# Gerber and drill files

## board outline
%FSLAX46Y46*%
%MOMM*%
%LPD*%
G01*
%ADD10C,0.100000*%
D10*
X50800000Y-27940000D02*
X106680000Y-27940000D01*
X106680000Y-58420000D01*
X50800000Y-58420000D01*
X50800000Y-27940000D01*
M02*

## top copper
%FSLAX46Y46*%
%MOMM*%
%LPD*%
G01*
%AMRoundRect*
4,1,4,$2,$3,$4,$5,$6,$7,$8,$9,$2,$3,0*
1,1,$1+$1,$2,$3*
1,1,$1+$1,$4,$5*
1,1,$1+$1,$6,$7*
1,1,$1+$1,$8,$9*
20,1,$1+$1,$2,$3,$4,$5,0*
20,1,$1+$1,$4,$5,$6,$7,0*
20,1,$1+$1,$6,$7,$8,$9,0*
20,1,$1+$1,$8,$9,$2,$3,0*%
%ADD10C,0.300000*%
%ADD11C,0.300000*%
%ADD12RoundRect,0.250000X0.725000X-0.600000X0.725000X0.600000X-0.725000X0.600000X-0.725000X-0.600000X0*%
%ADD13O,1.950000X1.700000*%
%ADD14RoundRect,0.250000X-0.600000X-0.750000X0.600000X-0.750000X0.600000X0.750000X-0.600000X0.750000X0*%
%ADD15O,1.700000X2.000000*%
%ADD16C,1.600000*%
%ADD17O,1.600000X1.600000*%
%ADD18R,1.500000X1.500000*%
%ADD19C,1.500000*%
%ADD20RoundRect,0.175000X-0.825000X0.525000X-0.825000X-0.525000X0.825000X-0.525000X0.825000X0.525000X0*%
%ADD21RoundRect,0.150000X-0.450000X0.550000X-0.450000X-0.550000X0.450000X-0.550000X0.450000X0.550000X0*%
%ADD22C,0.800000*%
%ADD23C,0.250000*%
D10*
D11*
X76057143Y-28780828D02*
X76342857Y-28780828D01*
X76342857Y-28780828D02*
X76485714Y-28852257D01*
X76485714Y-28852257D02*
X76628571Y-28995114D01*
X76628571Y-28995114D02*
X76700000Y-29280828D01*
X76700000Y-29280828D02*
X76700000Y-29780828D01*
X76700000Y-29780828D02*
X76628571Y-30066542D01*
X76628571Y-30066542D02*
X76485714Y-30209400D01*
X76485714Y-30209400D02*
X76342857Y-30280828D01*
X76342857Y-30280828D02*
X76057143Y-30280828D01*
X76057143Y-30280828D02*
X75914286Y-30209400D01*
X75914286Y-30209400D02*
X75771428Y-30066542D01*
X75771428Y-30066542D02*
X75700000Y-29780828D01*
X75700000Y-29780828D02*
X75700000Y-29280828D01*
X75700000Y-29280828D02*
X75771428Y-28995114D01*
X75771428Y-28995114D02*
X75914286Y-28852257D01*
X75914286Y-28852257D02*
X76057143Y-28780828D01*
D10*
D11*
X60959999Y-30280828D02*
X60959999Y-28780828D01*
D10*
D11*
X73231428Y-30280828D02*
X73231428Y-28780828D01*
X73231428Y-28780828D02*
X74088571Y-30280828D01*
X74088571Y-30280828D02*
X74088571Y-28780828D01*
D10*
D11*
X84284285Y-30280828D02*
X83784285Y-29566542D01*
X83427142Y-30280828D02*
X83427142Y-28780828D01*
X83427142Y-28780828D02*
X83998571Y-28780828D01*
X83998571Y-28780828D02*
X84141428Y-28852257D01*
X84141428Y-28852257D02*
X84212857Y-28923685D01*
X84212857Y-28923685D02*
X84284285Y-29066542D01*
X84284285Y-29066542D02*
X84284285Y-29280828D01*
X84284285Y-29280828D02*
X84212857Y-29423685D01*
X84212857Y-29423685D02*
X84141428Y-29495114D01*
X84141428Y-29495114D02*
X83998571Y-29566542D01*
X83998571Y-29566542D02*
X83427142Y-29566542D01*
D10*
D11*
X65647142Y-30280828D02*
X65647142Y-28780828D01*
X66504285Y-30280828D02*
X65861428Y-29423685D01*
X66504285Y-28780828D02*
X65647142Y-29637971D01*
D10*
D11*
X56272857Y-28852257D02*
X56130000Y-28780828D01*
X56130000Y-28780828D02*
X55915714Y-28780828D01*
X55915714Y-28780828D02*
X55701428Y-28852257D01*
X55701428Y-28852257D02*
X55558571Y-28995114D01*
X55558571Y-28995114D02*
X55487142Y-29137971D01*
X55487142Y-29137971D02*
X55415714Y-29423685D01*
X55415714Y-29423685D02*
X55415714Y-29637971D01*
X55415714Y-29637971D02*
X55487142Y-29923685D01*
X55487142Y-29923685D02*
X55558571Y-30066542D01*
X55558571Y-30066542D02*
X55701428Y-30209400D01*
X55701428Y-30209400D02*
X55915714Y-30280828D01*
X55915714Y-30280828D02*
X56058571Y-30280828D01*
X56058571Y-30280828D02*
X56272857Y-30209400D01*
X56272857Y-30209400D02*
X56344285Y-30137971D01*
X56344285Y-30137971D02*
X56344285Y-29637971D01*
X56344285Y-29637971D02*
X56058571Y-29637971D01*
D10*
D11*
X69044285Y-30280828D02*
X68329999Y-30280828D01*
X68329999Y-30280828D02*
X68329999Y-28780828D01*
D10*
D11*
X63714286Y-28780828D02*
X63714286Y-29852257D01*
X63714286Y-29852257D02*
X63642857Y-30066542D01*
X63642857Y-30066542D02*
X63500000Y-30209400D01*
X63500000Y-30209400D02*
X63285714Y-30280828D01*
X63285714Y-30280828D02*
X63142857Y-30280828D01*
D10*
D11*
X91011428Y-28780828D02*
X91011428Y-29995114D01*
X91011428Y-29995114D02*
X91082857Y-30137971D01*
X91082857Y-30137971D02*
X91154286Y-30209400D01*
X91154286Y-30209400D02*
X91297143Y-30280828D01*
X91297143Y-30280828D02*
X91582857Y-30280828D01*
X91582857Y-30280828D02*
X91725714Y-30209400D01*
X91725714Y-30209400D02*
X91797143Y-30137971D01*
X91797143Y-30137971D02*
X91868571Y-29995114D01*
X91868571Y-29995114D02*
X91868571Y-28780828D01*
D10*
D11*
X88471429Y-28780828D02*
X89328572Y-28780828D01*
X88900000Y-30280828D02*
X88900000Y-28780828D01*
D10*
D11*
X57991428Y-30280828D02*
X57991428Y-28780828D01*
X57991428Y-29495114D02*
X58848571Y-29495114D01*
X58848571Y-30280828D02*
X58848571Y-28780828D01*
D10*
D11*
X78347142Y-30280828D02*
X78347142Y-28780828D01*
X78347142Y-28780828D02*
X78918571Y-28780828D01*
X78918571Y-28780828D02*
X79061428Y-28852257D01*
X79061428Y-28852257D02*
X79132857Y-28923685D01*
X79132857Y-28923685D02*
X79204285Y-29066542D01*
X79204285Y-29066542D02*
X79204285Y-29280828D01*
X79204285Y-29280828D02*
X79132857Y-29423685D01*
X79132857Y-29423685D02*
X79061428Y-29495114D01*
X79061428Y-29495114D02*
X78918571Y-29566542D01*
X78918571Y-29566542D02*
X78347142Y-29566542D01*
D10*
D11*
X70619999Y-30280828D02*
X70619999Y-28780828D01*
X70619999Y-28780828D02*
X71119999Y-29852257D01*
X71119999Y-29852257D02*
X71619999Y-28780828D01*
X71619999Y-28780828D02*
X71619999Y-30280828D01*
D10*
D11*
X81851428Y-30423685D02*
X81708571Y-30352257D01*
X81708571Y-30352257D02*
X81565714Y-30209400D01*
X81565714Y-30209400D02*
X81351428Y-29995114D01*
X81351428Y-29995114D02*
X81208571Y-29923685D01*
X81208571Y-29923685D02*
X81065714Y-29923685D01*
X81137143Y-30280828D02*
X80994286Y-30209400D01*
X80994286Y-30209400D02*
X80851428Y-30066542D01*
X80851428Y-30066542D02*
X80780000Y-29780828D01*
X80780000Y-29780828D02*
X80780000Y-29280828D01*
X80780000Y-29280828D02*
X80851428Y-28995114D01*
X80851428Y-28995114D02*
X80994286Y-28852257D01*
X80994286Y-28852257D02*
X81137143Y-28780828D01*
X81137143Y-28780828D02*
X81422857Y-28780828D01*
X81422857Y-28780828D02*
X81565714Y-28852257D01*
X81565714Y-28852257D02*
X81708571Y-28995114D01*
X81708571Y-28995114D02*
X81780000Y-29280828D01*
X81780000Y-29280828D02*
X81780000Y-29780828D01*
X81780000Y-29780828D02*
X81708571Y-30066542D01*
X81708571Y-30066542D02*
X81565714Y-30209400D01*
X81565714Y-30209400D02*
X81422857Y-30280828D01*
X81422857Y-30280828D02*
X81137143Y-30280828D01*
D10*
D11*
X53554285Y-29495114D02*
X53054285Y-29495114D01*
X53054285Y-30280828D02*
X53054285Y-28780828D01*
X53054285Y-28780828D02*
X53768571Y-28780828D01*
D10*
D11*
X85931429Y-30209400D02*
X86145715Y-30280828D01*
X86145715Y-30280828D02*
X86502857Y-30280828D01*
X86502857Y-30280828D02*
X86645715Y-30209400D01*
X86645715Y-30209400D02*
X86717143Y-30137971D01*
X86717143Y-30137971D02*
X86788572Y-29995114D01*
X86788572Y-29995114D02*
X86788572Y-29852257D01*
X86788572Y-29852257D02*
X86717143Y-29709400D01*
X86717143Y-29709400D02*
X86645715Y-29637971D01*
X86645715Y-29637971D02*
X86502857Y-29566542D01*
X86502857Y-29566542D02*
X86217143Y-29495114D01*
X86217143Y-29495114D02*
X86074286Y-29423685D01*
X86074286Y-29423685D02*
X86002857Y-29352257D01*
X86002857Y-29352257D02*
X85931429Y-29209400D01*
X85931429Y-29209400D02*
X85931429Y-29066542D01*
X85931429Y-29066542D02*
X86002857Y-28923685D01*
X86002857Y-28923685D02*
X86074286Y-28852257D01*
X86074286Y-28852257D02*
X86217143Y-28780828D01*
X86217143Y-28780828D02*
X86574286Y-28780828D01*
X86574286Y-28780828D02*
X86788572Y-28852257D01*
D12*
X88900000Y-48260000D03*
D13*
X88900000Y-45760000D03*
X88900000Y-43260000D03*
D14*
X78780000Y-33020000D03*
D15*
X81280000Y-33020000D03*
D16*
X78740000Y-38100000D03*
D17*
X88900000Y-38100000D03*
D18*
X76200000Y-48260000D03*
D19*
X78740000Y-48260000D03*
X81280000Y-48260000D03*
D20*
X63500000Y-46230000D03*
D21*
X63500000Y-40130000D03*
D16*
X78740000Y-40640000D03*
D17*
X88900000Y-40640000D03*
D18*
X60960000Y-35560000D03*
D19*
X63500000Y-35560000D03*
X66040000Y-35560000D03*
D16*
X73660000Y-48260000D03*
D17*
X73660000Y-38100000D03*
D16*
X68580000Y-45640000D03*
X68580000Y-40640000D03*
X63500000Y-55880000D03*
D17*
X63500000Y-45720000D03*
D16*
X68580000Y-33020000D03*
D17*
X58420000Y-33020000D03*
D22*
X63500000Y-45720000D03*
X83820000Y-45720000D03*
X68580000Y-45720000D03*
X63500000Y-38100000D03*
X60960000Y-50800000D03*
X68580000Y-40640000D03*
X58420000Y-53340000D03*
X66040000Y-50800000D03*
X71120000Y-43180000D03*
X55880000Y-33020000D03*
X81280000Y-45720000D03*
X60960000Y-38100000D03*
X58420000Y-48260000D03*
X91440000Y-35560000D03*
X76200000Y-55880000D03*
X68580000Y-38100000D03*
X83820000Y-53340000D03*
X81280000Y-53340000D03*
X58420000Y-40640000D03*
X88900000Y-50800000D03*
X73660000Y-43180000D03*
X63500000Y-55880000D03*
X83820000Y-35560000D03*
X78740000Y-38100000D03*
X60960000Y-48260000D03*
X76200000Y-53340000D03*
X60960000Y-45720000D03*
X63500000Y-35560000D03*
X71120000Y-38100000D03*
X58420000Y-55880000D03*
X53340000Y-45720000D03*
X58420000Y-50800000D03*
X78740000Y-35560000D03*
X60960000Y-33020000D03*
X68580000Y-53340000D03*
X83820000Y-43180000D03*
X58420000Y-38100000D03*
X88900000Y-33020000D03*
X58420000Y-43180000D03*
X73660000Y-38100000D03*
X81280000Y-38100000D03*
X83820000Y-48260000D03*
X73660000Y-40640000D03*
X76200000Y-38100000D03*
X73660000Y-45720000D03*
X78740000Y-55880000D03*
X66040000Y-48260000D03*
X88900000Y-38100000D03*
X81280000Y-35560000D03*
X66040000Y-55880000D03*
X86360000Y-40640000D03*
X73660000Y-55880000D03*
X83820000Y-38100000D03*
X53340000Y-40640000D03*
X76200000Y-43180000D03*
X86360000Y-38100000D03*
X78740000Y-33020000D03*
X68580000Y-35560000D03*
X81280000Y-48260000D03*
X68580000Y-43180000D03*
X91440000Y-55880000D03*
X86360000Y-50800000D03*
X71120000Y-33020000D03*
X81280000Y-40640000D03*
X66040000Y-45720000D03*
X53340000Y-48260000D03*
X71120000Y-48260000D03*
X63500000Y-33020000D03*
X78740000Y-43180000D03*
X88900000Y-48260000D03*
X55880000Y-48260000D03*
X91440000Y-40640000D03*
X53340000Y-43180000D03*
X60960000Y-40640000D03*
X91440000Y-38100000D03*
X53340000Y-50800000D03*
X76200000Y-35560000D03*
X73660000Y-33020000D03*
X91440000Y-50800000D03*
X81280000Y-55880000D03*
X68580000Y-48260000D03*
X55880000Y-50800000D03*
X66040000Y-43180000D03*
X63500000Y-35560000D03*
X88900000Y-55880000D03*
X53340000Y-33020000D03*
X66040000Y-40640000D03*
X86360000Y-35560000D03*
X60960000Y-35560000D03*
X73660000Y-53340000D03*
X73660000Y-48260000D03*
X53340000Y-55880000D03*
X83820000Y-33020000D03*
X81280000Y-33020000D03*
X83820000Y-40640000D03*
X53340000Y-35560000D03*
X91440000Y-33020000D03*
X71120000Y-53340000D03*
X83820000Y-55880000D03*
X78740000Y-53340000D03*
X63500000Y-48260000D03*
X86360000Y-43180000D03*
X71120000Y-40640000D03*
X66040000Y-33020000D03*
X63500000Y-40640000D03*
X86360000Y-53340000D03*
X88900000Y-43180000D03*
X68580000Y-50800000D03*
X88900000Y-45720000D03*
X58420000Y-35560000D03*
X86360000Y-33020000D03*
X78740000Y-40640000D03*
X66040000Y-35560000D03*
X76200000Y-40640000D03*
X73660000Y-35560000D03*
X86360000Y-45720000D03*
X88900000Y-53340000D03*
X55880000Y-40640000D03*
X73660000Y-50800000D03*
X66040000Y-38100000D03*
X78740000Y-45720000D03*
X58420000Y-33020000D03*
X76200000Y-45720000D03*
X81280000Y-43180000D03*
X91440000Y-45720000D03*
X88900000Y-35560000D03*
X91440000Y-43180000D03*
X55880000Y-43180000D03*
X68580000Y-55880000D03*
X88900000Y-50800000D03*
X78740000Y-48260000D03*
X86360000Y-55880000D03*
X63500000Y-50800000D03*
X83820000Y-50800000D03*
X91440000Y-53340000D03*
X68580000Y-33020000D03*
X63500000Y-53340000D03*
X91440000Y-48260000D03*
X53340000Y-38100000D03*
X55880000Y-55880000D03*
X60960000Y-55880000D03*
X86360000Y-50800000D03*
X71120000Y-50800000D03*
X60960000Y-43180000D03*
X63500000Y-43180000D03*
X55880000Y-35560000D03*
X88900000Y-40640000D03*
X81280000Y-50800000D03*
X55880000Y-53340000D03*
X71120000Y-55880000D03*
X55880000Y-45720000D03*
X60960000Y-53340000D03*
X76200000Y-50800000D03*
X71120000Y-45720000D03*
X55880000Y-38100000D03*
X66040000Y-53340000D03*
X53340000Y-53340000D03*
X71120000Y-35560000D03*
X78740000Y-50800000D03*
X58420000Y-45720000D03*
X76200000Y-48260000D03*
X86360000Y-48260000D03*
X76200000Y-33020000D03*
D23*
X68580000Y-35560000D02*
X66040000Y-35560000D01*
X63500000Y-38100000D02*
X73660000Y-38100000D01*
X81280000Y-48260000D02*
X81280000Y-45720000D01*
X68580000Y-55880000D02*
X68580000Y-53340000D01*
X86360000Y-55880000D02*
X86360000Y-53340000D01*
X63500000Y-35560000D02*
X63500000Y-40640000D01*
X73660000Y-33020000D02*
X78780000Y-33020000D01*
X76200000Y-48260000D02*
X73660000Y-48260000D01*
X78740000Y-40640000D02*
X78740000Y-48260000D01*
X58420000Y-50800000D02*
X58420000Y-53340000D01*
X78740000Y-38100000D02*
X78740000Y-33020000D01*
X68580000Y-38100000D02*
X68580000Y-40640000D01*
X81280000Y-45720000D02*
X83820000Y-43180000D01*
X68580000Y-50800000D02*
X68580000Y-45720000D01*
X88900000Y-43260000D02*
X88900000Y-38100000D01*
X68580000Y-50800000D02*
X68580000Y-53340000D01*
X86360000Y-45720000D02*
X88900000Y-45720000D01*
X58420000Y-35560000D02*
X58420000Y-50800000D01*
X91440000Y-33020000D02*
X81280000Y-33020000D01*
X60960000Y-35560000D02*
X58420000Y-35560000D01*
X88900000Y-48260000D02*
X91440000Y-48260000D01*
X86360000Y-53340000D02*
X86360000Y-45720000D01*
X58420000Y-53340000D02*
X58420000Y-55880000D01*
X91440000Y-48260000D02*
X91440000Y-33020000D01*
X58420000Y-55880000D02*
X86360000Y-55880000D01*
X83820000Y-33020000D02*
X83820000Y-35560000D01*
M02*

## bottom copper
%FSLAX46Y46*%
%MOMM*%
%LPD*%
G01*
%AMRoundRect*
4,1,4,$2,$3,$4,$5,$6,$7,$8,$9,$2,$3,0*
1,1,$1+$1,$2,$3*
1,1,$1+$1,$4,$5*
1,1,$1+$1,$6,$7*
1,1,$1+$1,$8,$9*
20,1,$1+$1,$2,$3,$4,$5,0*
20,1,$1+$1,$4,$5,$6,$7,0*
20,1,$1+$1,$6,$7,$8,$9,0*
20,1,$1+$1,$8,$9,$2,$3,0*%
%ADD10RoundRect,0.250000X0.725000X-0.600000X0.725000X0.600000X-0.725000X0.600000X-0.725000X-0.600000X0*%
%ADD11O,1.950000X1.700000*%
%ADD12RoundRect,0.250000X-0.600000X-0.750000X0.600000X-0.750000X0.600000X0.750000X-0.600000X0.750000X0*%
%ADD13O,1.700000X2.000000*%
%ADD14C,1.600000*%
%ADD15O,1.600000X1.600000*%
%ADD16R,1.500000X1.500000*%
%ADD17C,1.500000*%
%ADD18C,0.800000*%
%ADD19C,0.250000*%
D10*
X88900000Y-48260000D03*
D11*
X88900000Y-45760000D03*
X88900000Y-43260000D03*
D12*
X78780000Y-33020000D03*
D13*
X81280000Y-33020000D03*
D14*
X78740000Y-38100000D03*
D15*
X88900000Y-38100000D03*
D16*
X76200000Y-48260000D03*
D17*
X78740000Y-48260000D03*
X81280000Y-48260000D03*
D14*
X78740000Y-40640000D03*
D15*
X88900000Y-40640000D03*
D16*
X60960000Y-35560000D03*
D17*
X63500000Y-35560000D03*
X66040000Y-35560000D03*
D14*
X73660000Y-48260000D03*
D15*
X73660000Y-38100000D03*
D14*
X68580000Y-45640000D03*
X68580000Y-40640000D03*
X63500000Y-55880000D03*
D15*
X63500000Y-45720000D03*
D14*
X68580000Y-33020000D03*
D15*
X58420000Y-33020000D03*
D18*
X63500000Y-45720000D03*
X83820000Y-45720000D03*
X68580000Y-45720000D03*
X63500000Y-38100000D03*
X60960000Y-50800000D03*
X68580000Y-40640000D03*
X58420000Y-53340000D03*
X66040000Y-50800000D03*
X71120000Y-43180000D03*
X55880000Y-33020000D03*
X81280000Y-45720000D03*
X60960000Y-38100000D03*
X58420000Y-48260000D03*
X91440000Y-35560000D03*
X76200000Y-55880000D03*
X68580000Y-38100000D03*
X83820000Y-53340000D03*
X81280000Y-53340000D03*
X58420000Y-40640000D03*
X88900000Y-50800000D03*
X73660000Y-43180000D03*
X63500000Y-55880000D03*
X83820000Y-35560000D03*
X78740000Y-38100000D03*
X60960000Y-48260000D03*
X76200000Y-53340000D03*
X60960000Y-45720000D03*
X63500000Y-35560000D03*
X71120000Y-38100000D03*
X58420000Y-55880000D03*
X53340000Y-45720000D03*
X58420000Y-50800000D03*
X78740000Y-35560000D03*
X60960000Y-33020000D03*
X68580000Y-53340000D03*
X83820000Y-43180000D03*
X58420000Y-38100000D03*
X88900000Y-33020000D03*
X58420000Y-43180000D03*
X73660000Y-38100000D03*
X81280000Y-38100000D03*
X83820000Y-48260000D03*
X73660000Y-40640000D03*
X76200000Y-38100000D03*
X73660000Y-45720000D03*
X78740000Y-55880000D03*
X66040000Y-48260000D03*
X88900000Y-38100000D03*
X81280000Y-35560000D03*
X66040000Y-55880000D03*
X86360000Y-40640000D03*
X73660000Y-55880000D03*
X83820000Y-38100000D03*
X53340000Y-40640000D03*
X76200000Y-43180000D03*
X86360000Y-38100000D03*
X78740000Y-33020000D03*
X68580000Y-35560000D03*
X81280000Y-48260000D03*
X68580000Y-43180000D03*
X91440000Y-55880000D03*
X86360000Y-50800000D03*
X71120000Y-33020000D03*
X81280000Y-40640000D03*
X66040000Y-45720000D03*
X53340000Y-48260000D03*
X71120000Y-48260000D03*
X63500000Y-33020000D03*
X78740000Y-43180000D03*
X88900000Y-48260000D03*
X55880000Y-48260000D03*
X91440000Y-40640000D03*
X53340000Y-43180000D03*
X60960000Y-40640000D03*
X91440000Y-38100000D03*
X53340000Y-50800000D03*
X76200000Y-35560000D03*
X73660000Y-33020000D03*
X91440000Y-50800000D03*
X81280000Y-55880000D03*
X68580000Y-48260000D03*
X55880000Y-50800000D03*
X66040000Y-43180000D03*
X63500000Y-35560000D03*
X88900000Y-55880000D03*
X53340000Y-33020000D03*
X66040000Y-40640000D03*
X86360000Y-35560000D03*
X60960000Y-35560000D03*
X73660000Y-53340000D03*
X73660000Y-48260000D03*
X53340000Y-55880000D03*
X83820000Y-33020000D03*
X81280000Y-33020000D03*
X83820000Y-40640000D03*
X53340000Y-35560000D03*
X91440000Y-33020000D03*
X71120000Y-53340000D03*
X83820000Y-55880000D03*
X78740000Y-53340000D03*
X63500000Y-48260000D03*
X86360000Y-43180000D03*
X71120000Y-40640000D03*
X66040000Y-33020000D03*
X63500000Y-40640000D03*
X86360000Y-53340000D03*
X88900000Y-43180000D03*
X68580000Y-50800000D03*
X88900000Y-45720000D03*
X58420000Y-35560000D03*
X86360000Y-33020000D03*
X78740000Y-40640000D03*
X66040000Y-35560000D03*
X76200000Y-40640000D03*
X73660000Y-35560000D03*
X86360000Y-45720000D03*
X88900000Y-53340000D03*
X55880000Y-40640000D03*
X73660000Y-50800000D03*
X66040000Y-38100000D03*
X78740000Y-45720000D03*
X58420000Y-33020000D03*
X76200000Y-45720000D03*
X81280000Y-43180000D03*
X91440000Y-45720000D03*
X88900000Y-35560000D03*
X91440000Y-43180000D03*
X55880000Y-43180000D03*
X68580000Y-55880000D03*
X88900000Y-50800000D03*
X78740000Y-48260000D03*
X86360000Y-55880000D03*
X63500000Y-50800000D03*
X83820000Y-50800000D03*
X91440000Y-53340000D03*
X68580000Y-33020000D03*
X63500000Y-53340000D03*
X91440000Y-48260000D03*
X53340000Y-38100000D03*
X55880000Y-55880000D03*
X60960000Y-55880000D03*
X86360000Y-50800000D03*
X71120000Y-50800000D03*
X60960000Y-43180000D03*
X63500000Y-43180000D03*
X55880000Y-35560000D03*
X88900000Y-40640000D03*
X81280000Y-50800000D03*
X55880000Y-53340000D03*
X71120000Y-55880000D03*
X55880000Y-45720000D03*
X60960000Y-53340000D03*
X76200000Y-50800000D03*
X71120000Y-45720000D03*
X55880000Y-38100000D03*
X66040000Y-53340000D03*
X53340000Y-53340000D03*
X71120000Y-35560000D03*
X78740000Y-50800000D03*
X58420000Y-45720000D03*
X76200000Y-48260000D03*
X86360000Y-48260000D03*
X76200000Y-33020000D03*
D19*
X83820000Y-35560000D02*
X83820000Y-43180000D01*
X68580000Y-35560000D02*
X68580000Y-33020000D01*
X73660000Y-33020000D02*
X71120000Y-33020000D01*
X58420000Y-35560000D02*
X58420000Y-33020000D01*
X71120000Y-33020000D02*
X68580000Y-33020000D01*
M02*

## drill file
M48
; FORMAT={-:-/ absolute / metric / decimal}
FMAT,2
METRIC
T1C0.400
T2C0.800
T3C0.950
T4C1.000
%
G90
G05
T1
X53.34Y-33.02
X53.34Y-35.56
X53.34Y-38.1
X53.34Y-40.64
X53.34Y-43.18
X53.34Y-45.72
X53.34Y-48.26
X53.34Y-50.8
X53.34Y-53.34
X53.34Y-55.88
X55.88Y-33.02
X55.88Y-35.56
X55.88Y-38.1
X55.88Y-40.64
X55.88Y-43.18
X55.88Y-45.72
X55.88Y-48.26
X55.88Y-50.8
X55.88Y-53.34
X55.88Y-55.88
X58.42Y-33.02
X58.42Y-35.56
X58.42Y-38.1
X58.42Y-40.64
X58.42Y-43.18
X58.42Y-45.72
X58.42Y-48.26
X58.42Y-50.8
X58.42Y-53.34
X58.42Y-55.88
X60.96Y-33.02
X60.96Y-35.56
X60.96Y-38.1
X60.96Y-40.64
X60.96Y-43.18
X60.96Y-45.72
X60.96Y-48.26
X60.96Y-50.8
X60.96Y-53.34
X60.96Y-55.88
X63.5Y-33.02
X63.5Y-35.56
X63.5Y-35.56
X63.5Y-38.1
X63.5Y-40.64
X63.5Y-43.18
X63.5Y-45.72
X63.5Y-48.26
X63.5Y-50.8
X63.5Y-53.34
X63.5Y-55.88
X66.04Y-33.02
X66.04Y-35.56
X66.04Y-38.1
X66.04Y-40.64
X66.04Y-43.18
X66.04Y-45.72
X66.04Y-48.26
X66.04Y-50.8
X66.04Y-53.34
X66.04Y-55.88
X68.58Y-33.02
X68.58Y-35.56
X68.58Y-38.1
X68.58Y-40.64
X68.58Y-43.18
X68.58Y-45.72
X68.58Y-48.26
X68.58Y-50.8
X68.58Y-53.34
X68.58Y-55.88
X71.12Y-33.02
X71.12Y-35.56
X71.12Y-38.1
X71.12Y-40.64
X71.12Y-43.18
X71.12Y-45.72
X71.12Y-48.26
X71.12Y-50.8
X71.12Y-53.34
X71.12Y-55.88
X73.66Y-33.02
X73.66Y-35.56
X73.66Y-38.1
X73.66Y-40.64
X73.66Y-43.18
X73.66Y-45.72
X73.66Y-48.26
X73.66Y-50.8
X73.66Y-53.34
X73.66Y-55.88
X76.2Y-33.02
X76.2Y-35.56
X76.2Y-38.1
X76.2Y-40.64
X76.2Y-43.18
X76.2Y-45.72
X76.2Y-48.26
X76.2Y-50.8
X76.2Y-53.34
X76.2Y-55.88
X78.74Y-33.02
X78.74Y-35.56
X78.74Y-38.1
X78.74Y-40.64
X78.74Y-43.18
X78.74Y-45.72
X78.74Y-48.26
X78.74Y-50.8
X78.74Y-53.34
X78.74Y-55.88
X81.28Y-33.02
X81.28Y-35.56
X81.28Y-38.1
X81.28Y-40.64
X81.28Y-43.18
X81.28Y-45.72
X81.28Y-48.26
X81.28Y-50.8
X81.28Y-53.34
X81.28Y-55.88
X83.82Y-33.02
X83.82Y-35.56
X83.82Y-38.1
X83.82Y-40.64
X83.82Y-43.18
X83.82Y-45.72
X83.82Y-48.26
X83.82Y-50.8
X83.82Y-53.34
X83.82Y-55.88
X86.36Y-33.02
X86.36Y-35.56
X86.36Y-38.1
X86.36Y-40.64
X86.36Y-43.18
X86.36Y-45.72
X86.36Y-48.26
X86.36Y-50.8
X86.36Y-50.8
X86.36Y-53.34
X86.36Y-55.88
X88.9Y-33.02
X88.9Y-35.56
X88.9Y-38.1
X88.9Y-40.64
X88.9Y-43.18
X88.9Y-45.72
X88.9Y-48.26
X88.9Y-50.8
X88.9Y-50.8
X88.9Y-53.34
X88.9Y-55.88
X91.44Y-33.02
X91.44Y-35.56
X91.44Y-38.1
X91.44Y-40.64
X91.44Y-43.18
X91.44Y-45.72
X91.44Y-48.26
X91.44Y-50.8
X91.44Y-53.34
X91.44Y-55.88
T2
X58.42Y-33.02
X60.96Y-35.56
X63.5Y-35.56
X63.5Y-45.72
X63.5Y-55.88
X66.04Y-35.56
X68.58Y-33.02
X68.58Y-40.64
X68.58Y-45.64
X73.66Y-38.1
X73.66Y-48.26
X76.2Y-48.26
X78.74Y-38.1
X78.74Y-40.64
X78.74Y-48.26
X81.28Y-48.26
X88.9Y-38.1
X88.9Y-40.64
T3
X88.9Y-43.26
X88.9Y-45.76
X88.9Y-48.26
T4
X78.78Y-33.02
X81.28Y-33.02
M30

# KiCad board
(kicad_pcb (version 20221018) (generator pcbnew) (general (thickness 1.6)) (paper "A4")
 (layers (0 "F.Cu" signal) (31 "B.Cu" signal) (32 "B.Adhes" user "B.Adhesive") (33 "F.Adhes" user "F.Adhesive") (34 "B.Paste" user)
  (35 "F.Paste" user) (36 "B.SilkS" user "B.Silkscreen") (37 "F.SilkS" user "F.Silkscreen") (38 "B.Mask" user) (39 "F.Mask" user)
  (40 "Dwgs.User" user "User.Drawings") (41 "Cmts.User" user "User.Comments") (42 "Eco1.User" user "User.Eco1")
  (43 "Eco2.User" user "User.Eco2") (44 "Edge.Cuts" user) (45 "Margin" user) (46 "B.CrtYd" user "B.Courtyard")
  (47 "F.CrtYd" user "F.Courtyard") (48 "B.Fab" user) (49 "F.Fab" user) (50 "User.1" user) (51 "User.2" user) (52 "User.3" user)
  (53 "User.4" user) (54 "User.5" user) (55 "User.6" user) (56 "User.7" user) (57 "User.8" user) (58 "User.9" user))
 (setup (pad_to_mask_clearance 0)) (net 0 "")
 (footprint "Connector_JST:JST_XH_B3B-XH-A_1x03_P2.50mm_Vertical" (layer "F.Cu") (at 88.9 48.26 90)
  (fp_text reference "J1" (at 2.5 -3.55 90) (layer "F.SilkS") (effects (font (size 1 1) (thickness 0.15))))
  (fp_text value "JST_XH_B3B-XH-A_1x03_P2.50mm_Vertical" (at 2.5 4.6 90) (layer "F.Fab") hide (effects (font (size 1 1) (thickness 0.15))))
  (pad "1" thru_hole roundrect (at 0 0 90) (size 1.7 1.95) (drill 0.95) (layers "*.Cu" "*.Mask") (roundrect_rratio 0.147059))
  (pad "2" thru_hole oval (at 2.5 0 90) (size 1.7 1.95) (drill 0.95) (layers "*.Cu" "*.Mask"))
  (pad "3" thru_hole oval (at 5 0 90) (size 1.7 1.95) (drill 0.95) (layers "*.Cu" "*.Mask")))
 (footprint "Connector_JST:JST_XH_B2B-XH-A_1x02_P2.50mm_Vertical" (layer "F.Cu") (at 78.78 33.02)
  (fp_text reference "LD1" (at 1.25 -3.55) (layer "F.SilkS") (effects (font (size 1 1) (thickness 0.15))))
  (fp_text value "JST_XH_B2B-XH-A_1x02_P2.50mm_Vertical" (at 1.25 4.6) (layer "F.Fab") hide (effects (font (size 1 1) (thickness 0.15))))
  (pad "1" thru_hole roundrect (at 0 0) (size 1.7 2) (drill 1) (layers "*.Cu" "*.Mask") (roundrect_rratio 0.147059))
  (pad "2" thru_hole oval (at 2.5 0) (size 1.7 2) (drill 1) (layers "*.Cu" "*.Mask")))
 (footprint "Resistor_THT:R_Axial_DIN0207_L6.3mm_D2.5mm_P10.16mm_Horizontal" (layer "F.Cu") (at 78.74 38.1)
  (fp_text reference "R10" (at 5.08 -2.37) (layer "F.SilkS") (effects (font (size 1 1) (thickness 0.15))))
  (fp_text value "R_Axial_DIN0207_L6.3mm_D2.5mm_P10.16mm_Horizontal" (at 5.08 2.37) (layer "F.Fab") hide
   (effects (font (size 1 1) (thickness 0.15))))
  (pad "1" thru_hole circle (at 0 0) (size 1.6 1.6) (drill 0.8) (layers "*.Cu" "*.Mask"))
  (pad "2" thru_hole oval (at 10.16 0) (size 1.6 1.6) (drill 0.8) (layers "*.Cu" "*.Mask")))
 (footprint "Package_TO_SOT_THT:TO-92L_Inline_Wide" (layer "F.Cu") (at 76.2 48.26)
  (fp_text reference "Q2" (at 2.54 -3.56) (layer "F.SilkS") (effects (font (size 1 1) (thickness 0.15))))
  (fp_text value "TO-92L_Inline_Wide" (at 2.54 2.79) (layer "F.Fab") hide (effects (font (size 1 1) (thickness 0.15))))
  (pad "1" thru_hole rect (at 0 0) (size 1.5 1.5) (drill 0.8) (layers "*.Cu" "*.Mask"))
  (pad "2" thru_hole circle (at 2.54 0) (size 1.5 1.5) (drill 0.8) (layers "*.Cu" "*.Mask"))
  (pad "3" thru_hole circle (at 5.08 0) (size 1.5 1.5) (drill 0.8) (layers "*.Cu" "*.Mask")))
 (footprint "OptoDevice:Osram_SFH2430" (layer "F.Cu") (at 63.5 43.18 90)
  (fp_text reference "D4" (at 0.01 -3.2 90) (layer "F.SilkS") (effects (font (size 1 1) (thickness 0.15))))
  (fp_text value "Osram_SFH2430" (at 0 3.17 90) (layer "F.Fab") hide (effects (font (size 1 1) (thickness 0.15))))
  (pad "" smd roundrect (at -3.05 0 270) (size 1.3 1.9) (layers "F.Paste") (roundrect_rratio 0.125))
  (pad "" smd roundrect (at -3.05 0 270) (size 1.5 2.1) (layers "F.Mask") (roundrect_rratio 0.125))
  (pad "" smd roundrect (at 3.05 0 270) (size 1.3 1.1) (layers "F.Paste") (roundrect_rratio 0.125))
  (pad "" smd roundrect (at 3.05 0 270) (size 1.5 1.3) (layers "F.Mask") (roundrect_rratio 0.125))
  (pad "1" smd roundrect (at -3.05 0 270) (size 1.4 2) (layers "F.Cu" "F.Mask") (roundrect_rratio 0.125))
  (pad "2" smd roundrect (at 3.05 0 270) (size 1.4 1.2) (layers "F.Cu" "F.Mask") (roundrect_rratio 0.125)))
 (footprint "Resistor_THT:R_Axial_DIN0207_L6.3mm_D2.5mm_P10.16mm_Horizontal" (layer "F.Cu") (at 78.74 40.64)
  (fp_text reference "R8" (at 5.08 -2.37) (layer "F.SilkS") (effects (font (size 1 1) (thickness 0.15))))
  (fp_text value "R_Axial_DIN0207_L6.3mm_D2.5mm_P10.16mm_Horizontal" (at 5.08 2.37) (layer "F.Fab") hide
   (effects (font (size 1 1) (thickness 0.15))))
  (pad "1" thru_hole circle (at 0 0) (size 1.6 1.6) (drill 0.8) (layers "*.Cu" "*.Mask"))
  (pad "2" thru_hole oval (at 10.16 0) (size 1.6 1.6) (drill 0.8) (layers "*.Cu" "*.Mask")))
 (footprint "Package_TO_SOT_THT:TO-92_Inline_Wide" (layer "F.Cu") (at 60.96 35.56)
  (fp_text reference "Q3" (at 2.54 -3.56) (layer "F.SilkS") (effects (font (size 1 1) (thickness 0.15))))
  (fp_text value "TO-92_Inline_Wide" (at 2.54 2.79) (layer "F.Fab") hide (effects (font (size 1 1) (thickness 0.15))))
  (pad "1" thru_hole rect (at 0 0) (size 1.5 1.5) (drill 0.8) (layers "*.Cu" "*.Mask"))
  (pad "2" thru_hole circle (at 2.54 0) (size 1.5 1.5) (drill 0.8) (layers "*.Cu" "*.Mask"))
  (pad "3" thru_hole circle (at 5.08 0) (size 1.5 1.5) (drill 0.8) (layers "*.Cu" "*.Mask")))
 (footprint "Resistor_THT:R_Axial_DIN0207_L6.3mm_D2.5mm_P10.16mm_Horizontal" (layer "B.Cu") (at 73.66 48.26 90)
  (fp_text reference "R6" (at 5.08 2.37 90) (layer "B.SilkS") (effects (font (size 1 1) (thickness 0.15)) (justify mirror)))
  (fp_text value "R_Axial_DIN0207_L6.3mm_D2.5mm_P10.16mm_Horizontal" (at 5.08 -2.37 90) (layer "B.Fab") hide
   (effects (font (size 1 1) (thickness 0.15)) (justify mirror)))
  (pad "1" thru_hole circle (at 0 0 90) (size 1.6 1.6) (drill 0.8) (layers "*.Cu" "*.Mask"))
  (pad "2" thru_hole oval (at 10.16 0 90) (size 1.6 1.6) (drill 0.8) (layers "*.Cu" "*.Mask")))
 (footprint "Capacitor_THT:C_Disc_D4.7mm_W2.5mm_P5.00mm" (layer "B.Cu") (at 68.58 45.64 90)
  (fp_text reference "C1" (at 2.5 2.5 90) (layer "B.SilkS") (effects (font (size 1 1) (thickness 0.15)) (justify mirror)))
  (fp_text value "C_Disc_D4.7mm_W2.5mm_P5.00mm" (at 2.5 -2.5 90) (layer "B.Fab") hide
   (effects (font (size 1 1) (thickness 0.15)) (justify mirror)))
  (pad "1" thru_hole circle (at 0 0 90) (size 1.6 1.6) (drill 0.8) (layers "*.Cu" "*.Mask"))
  (pad "2" thru_hole circle (at 5 0 90) (size 1.6 1.6) (drill 0.8) (layers "*.Cu" "*.Mask")))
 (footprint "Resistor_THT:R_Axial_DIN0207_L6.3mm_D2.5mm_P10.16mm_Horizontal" (layer "B.Cu") (at 63.5 55.88 90)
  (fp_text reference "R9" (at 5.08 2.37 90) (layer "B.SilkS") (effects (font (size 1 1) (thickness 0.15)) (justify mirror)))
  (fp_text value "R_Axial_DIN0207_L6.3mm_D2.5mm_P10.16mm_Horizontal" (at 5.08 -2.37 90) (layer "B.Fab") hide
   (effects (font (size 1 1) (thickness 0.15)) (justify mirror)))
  (pad "1" thru_hole circle (at 0 0 90) (size 1.6 1.6) (drill 0.8) (layers "*.Cu" "*.Mask"))
  (pad "2" thru_hole oval (at 10.16 0 90) (size 1.6 1.6) (drill 0.8) (layers "*.Cu" "*.Mask")))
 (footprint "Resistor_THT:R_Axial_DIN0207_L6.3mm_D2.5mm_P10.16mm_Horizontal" (layer "B.Cu") (at 68.58 33.02 180)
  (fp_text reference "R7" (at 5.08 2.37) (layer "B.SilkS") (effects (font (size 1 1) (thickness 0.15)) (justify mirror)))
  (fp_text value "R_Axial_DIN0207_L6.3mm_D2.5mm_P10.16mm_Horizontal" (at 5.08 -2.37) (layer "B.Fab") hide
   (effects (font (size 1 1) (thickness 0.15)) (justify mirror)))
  (pad "1" thru_hole circle (at 0 0 180) (size 1.6 1.6) (drill 0.8) (layers "*.Cu" "*.Mask"))
  (pad "2" thru_hole oval (at 10.16 0 180) (size 1.6 1.6) (drill 0.8) (layers "*.Cu" "*.Mask")))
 (gr_rect (start 50.8 27.94) (end 106.68 58.42) (stroke (width 0.1) (type default)) (fill none) (layer "Edge.Cuts"))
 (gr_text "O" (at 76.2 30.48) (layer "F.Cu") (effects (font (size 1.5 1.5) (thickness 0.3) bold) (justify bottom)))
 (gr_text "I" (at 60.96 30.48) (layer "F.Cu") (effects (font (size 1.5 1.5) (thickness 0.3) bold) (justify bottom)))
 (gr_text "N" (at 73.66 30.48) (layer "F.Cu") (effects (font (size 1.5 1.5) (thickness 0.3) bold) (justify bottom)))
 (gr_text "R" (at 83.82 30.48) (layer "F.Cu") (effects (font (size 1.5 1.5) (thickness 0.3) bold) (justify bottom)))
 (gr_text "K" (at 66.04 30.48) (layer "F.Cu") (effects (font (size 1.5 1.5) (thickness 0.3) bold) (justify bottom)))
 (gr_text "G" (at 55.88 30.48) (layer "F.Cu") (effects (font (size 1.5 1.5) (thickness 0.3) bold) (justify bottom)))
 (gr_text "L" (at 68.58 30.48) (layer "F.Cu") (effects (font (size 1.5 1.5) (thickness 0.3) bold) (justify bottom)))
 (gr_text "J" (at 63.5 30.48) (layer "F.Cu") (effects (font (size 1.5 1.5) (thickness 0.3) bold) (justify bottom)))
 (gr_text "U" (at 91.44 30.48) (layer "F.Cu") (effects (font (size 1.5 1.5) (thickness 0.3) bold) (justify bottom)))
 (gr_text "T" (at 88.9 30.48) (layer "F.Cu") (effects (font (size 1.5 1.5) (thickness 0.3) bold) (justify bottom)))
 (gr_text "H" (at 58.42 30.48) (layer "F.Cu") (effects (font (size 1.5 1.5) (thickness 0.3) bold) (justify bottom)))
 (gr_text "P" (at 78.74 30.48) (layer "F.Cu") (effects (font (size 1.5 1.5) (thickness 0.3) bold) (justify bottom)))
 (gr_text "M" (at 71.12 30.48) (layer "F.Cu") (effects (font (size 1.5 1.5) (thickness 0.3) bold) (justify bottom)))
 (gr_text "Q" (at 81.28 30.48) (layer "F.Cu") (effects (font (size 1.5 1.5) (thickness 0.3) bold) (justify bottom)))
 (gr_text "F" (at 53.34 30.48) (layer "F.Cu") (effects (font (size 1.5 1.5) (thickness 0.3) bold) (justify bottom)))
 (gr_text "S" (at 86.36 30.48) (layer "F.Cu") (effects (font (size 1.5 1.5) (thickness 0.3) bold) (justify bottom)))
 (segment (start 68.58 35.56) (end 66.04 35.56) (width 0.25) (layer "F.Cu") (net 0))
 (segment (start 63.5 38.1) (end 73.66 38.1) (width 0.25) (layer "F.Cu") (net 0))
 (segment (start 81.28 48.26) (end 81.28 45.72) (width 0.25) (layer "F.Cu") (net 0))
 (segment (start 68.58 55.88) (end 68.58 53.34) (width 0.25) (layer "F.Cu") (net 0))
 (segment (start 86.36 55.88) (end 86.36 53.34) (width 0.25) (layer "F.Cu") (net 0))
 (segment (start 63.5 35.56) (end 63.5 40.64) (width 0.25) (layer "F.Cu") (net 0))
 (segment (start 73.66 33.02) (end 78.78 33.02) (width 0.25) (layer "F.Cu") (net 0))
 (segment (start 76.2 48.26) (end 73.66 48.26) (width 0.25) (layer "F.Cu") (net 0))
 (segment (start 78.74 40.64) (end 78.74 48.26) (width 0.25) (layer "F.Cu") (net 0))
 (segment (start 58.42 50.8) (end 58.42 53.34) (width 0.25) (layer "F.Cu") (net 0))
 (segment (start 78.74 38.1) (end 78.74 33.02) (width 0.25) (layer "F.Cu") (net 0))
 (segment (start 68.58 38.1) (end 68.58 40.64) (width 0.25) (layer "F.Cu") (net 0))
 (segment (start 81.28 45.72) (end 83.82 43.18) (width 0.25) (layer "F.Cu") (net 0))
 (segment (start 68.58 50.8) (end 68.58 45.72) (width 0.25) (layer "F.Cu") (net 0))
 (segment (start 88.9 43.26) (end 88.9 38.1) (width 0.25) (layer "F.Cu") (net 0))
 (segment (start 68.58 50.8) (end 68.58 53.34) (width 0.25) (layer "F.Cu") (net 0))
 (segment (start 86.36 45.72) (end 88.9 45.72) (width 0.25) (layer "F.Cu") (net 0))
 (segment (start 58.42 35.56) (end 58.42 50.8) (width 0.25) (layer "F.Cu") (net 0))
 (segment (start 91.44 33.02) (end 81.28 33.02) (width 0.25) (layer "F.Cu") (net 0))
 (segment (start 60.96 35.56) (end 58.42 35.56) (width 0.25) (layer "F.Cu") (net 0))
 (segment (start 88.9 48.26) (end 91.44 48.26) (width 0.25) (layer "F.Cu") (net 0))
 (segment (start 86.36 53.34) (end 86.36 45.72) (width 0.25) (layer "F.Cu") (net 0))
 (segment (start 58.42 53.34) (end 58.42 55.88) (width 0.25) (layer "F.Cu") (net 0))
 (segment (start 91.44 48.26) (end 91.44 33.02) (width 0.25) (layer "F.Cu") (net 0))
 (segment (start 58.42 55.88) (end 86.36 55.88) (width 0.25) (layer "F.Cu") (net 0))
 (segment (start 83.82 33.02) (end 83.82 35.56) (width 0.25) (layer "F.Cu") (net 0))
 (via (at 63.5 45.72) (size 0.8) (drill 0.4) (layers "F.Cu" "B.Cu") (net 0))
 (via (at 83.82 45.72) (size 0.8) (drill 0.4) (layers "F.Cu" "B.Cu") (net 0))
 (via (at 68.58 45.72) (size 0.8) (drill 0.4) (layers "F.Cu" "B.Cu") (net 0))
 (via (at 63.5 38.1) (size 0.8) (drill 0.4) (layers "F.Cu" "B.Cu") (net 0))
 (via (at 60.96 50.8) (size 0.8) (drill 0.4) (layers "F.Cu" "B.Cu") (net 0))
 (via (at 68.58 40.64) (size 0.8) (drill 0.4) (layers "F.Cu" "B.Cu") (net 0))
 (via (at 58.42 53.34) (size 0.8) (drill 0.4) (layers "F.Cu" "B.Cu") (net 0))
 (via (at 66.04 50.8) (size 0.8) (drill 0.4) (layers "F.Cu" "B.Cu") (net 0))
 (via (at 71.12 43.18) (size 0.8) (drill 0.4) (layers "F.Cu" "B.Cu") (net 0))
 (via (at 55.88 33.02) (size 0.8) (drill 0.4) (layers "F.Cu" "B.Cu") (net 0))
 (via (at 81.28 45.72) (size 0.8) (drill 0.4) (layers "F.Cu" "B.Cu") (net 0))
 (via (at 60.96 38.1) (size 0.8) (drill 0.4) (layers "F.Cu" "B.Cu") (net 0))
 (via (at 58.42 48.26) (size 0.8) (drill 0.4) (layers "F.Cu" "B.Cu") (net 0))
 (via (at 91.44 35.56) (size 0.8) (drill 0.4) (layers "F.Cu" "B.Cu") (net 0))
 (via (at 76.2 55.88) (size 0.8) (drill 0.4) (layers "F.Cu" "B.Cu") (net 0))
 (via (at 68.58 38.1) (size 0.8) (drill 0.4) (layers "F.Cu" "B.Cu") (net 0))
 (via (at 83.82 53.34) (size 0.8) (drill 0.4) (layers "F.Cu" "B.Cu") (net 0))
 (via (at 81.28 53.34) (size 0.8) (drill 0.4) (layers "F.Cu" "B.Cu") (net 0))
 (via (at 58.42 40.64) (size 0.8) (drill 0.4) (layers "F.Cu" "B.Cu") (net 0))
 (via (at 88.9 50.8) (size 0.8) (drill 0.4) (layers "F.Cu" "B.Cu") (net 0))
 (via (at 73.66 43.18) (size 0.8) (drill 0.4) (layers "F.Cu" "B.Cu") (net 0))
 (via (at 63.5 55.88) (size 0.8) (drill 0.4) (layers "F.Cu" "B.Cu") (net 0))
 (via (at 83.82 35.56) (size 0.8) (drill 0.4) (layers "F.Cu" "B.Cu") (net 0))
 (via (at 78.74 38.1) (size 0.8) (drill 0.4) (layers "F.Cu" "B.Cu") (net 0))
 (via (at 60.96 48.26) (size 0.8) (drill 0.4) (layers "F.Cu" "B.Cu") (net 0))
 (via (at 76.2 53.34) (size 0.8) (drill 0.4) (layers "F.Cu" "B.Cu") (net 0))
 (via (at 60.96 45.72) (size 0.8) (drill 0.4) (layers "F.Cu" "B.Cu") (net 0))
 (via (at 63.5 35.56) (size 0.8) (drill 0.4) (layers "F.Cu" "B.Cu") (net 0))
 (via (at 71.12 38.1) (size 0.8) (drill 0.4) (layers "F.Cu" "B.Cu") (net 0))
 (via (at 58.42 55.88) (size 0.8) (drill 0.4) (layers "F.Cu" "B.Cu") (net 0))
 (via (at 53.34 45.72) (size 0.8) (drill 0.4) (layers "F.Cu" "B.Cu") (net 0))
 (via (at 58.42 50.8) (size 0.8) (drill 0.4) (layers "F.Cu" "B.Cu") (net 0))
 (via (at 78.74 35.56) (size 0.8) (drill 0.4) (layers "F.Cu" "B.Cu") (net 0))
 (via (at 60.96 33.02) (size 0.8) (drill 0.4) (layers "F.Cu" "B.Cu") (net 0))
 (via (at 68.58 53.34) (size 0.8) (drill 0.4) (layers "F.Cu" "B.Cu") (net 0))
 (via (at 83.82 43.18) (size 0.8) (drill 0.4) (layers "F.Cu" "B.Cu") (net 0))
 (via (at 58.42 38.1) (size 0.8) (drill 0.4) (layers "F.Cu" "B.Cu") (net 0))
 (via (at 88.9 33.02) (size 0.8) (drill 0.4) (layers "F.Cu" "B.Cu") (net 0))
 (via (at 58.42 43.18) (size 0.8) (drill 0.4) (layers "F.Cu" "B.Cu") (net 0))
 (via (at 73.66 38.1) (size 0.8) (drill 0.4) (layers "F.Cu" "B.Cu") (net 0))
 (via (at 81.28 38.1) (size 0.8) (drill 0.4) (layers "F.Cu" "B.Cu") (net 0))
 (via (at 83.82 48.26) (size 0.8) (drill 0.4) (layers "F.Cu" "B.Cu") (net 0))
 (via (at 73.66 40.64) (size 0.8) (drill 0.4) (layers "F.Cu" "B.Cu") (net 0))
 (via (at 76.2 38.1) (size 0.8) (drill 0.4) (layers "F.Cu" "B.Cu") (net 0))
 (via (at 73.66 45.72) (size 0.8) (drill 0.4) (layers "F.Cu" "B.Cu") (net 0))
 (via (at 78.74 55.88) (size 0.8) (drill 0.4) (layers "F.Cu" "B.Cu") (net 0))
 (via (at 66.04 48.26) (size 0.8) (drill 0.4) (layers "F.Cu" "B.Cu") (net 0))
 (via (at 88.9 38.1) (size 0.8) (drill 0.4) (layers "F.Cu" "B.Cu") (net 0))
 (via (at 81.28 35.56) (size 0.8) (drill 0.4) (layers "F.Cu" "B.Cu") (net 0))
 (via (at 66.04 55.88) (size 0.8) (drill 0.4) (layers "F.Cu" "B.Cu") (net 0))
 (via (at 86.36 40.64) (size 0.8) (drill 0.4) (layers "F.Cu" "B.Cu") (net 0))
 (via (at 73.66 55.88) (size 0.8) (drill 0.4) (layers "F.Cu" "B.Cu") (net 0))
 (via (at 83.82 38.1) (size 0.8) (drill 0.4) (layers "F.Cu" "B.Cu") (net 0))
 (via (at 53.34 40.64) (size 0.8) (drill 0.4) (layers "F.Cu" "B.Cu") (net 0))
 (via (at 76.2 43.18) (size 0.8) (drill 0.4) (layers "F.Cu" "B.Cu") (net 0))
 (via (at 86.36 38.1) (size 0.8) (drill 0.4) (layers "F.Cu" "B.Cu") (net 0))
 (via (at 78.74 33.02) (size 0.8) (drill 0.4) (layers "F.Cu" "B.Cu") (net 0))
 (via (at 68.58 35.56) (size 0.8) (drill 0.4) (layers "F.Cu" "B.Cu") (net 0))
 (via (at 81.28 48.26) (size 0.8) (drill 0.4) (layers "F.Cu" "B.Cu") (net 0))
 (via (at 68.58 43.18) (size 0.8) (drill 0.4) (layers "F.Cu" "B.Cu") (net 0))
 (via (at 91.44 55.88) (size 0.8) (drill 0.4) (layers "F.Cu" "B.Cu") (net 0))
 (via (at 86.36 50.8) (size 0.8) (drill 0.4) (layers "F.Cu" "B.Cu") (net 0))
 (via (at 71.12 33.02) (size 0.8) (drill 0.4) (layers "F.Cu" "B.Cu") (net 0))
 (via (at 81.28 40.64) (size 0.8) (drill 0.4) (layers "F.Cu" "B.Cu") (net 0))
 (via (at 66.04 45.72) (size 0.8) (drill 0.4) (layers "F.Cu" "B.Cu") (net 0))
 (via (at 53.34 48.26) (size 0.8) (drill 0.4) (layers "F.Cu" "B.Cu") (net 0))
 (via (at 71.12 48.26) (size 0.8) (drill 0.4) (layers "F.Cu" "B.Cu") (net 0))
 (via (at 63.5 33.02) (size 0.8) (drill 0.4) (layers "F.Cu" "B.Cu") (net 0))
 (via (at 78.74 43.18) (size 0.8) (drill 0.4) (layers "F.Cu" "B.Cu") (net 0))
 (via (at 88.9 48.26) (size 0.8) (drill 0.4) (layers "F.Cu" "B.Cu") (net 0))
 (via (at 55.88 48.26) (size 0.8) (drill 0.4) (layers "F.Cu" "B.Cu") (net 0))
 (via (at 91.44 40.64) (size 0.8) (drill 0.4) (layers "F.Cu" "B.Cu") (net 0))
 (via (at 53.34 43.18) (size 0.8) (drill 0.4) (layers "F.Cu" "B.Cu") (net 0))
 (via (at 60.96 40.64) (size 0.8) (drill 0.4) (layers "F.Cu" "B.Cu") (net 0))
 (via (at 91.44 38.1) (size 0.8) (drill 0.4) (layers "F.Cu" "B.Cu") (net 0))
 (via (at 53.34 50.8) (size 0.8) (drill 0.4) (layers "F.Cu" "B.Cu") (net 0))
 (via (at 76.2 35.56) (size 0.8) (drill 0.4) (layers "F.Cu" "B.Cu") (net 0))
 (via (at 73.66 33.02) (size 0.8) (drill 0.4) (layers "F.Cu" "B.Cu") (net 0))
 (via (at 91.44 50.8) (size 0.8) (drill 0.4) (layers "F.Cu" "B.Cu") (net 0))
 (via (at 81.28 55.88) (size 0.8) (drill 0.4) (layers "F.Cu" "B.Cu") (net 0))
 (via (at 68.58 48.26) (size 0.8) (drill 0.4) (layers "F.Cu" "B.Cu") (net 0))
 (via (at 55.88 50.8) (size 0.8) (drill 0.4) (layers "F.Cu" "B.Cu") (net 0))
 (via (at 66.04 43.18) (size 0.8) (drill 0.4) (layers "F.Cu" "B.Cu") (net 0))
 (via (at 63.5 35.56) (size 0.8) (drill 0.4) (layers "F.Cu" "B.Cu") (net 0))
 (via (at 88.9 55.88) (size 0.8) (drill 0.4) (layers "F.Cu" "B.Cu") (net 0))
 (via (at 53.34 33.02) (size 0.8) (drill 0.4) (layers "F.Cu" "B.Cu") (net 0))
 (via (at 66.04 40.64) (size 0.8) (drill 0.4) (layers "F.Cu" "B.Cu") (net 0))
 (via (at 86.36 35.56) (size 0.8) (drill 0.4) (layers "F.Cu" "B.Cu") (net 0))
 (via (at 60.96 35.56) (size 0.8) (drill 0.4) (layers "F.Cu" "B.Cu") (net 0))
 (via (at 73.66 53.34) (size 0.8) (drill 0.4) (layers "F.Cu" "B.Cu") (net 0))
 (via (at 73.66 48.26) (size 0.8) (drill 0.4) (layers "F.Cu" "B.Cu") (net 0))
 (via (at 53.34 55.88) (size 0.8) (drill 0.4) (layers "F.Cu" "B.Cu") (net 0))
 (via (at 83.82 33.02) (size 0.8) (drill 0.4) (layers "F.Cu" "B.Cu") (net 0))
 (via (at 81.28 33.02) (size 0.8) (drill 0.4) (layers "F.Cu" "B.Cu") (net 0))
 (via (at 83.82 40.64) (size 0.8) (drill 0.4) (layers "F.Cu" "B.Cu") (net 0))
 (via (at 53.34 35.56) (size 0.8) (drill 0.4) (layers "F.Cu" "B.Cu") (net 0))
 (via (at 91.44 33.02) (size 0.8) (drill 0.4) (layers "F.Cu" "B.Cu") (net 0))
 (via (at 71.12 53.34) (size 0.8) (drill 0.4) (layers "F.Cu" "B.Cu") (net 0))
 (via (at 83.82 55.88) (size 0.8) (drill 0.4) (layers "F.Cu" "B.Cu") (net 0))
 (via (at 78.74 53.34) (size 0.8) (drill 0.4) (layers "F.Cu" "B.Cu") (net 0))
 (via (at 63.5 48.26) (size 0.8) (drill 0.4) (layers "F.Cu" "B.Cu") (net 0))
 (via (at 86.36 43.18) (size 0.8) (drill 0.4) (layers "F.Cu" "B.Cu") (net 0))
 (via (at 71.12 40.64) (size 0.8) (drill 0.4) (layers "F.Cu" "B.Cu") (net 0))
 (via (at 66.04 33.02) (size 0.8) (drill 0.4) (layers "F.Cu" "B.Cu") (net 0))
 (via (at 63.5 40.64) (size 0.8) (drill 0.4) (layers "F.Cu" "B.Cu") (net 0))
 (via (at 86.36 53.34) (size 0.8) (drill 0.4) (layers "F.Cu" "B.Cu") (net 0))
 (via (at 88.9 43.18) (size 0.8) (drill 0.4) (layers "F.Cu" "B.Cu") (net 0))
 (via (at 68.58 50.8) (size 0.8) (drill 0.4) (layers "F.Cu" "B.Cu") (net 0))
 (via (at 88.9 45.72) (size 0.8) (drill 0.4) (layers "F.Cu" "B.Cu") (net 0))
 (via (at 58.42 35.56) (size 0.8) (drill 0.4) (layers "F.Cu" "B.Cu") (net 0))
 (via (at 86.36 33.02) (size 0.8) (drill 0.4) (layers "F.Cu" "B.Cu") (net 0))
 (via (at 78.74 40.64) (size 0.8) (drill 0.4) (layers "F.Cu" "B.Cu") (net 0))
 (via (at 66.04 35.56) (size 0.8) (drill 0.4) (layers "F.Cu" "B.Cu") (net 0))
 (via (at 76.2 40.64) (size 0.8) (drill 0.4) (layers "F.Cu" "B.Cu") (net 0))
 (via (at 73.66 35.56) (size 0.8) (drill 0.4) (layers "F.Cu" "B.Cu") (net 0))
 (via (at 86.36 45.72) (size 0.8) (drill 0.4) (layers "F.Cu" "B.Cu") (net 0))
 (via (at 88.9 53.34) (size 0.8) (drill 0.4) (layers "F.Cu" "B.Cu") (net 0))
 (via (at 55.88 40.64) (size 0.8) (drill 0.4) (layers "F.Cu" "B.Cu") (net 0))
 (via (at 73.66 50.8) (size 0.8) (drill 0.4) (layers "F.Cu" "B.Cu") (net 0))
 (via (at 66.04 38.1) (size 0.8) (drill 0.4) (layers "F.Cu" "B.Cu") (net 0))
 (via (at 78.74 45.72) (size 0.8) (drill 0.4) (layers "F.Cu" "B.Cu") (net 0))
 (via (at 58.42 33.02) (size 0.8) (drill 0.4) (layers "F.Cu" "B.Cu") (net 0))
 (via (at 76.2 45.72) (size 0.8) (drill 0.4) (layers "F.Cu" "B.Cu") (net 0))
 (via (at 81.28 43.18) (size 0.8) (drill 0.4) (layers "F.Cu" "B.Cu") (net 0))
 (via (at 91.44 45.72) (size 0.8) (drill 0.4) (layers "F.Cu" "B.Cu") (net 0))
 (via (at 88.9 35.56) (size 0.8) (drill 0.4) (layers "F.Cu" "B.Cu") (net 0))
 (via (at 91.44 43.18) (size 0.8) (drill 0.4) (layers "F.Cu" "B.Cu") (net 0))
 (via (at 55.88 43.18) (size 0.8) (drill 0.4) (layers "F.Cu" "B.Cu") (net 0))
 (via (at 68.58 55.88) (size 0.8) (drill 0.4) (layers "F.Cu" "B.Cu") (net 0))
 (via (at 88.9 50.8) (size 0.8) (drill 0.4) (layers "F.Cu" "B.Cu") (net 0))
 (via (at 78.74 48.26) (size 0.8) (drill 0.4) (layers "F.Cu" "B.Cu") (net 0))
 (via (at 86.36 55.88) (size 0.8) (drill 0.4) (layers "F.Cu" "B.Cu") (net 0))
 (via (at 63.5 50.8) (size 0.8) (drill 0.4) (layers "F.Cu" "B.Cu") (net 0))
 (via (at 83.82 50.8) (size 0.8) (drill 0.4) (layers "F.Cu" "B.Cu") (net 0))
 (via (at 91.44 53.34) (size 0.8) (drill 0.4) (layers "F.Cu" "B.Cu") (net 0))
 (via (at 68.58 33.02) (size 0.8) (drill 0.4) (layers "F.Cu" "B.Cu") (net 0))
 (via (at 63.5 53.34) (size 0.8) (drill 0.4) (layers "F.Cu" "B.Cu") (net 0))
 (via (at 91.44 48.26) (size 0.8) (drill 0.4) (layers "F.Cu" "B.Cu") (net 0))
 (via (at 53.34 38.1) (size 0.8) (drill 0.4) (layers "F.Cu" "B.Cu") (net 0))
 (via (at 55.88 55.88) (size 0.8) (drill 0.4) (layers "F.Cu" "B.Cu") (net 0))
 (via (at 60.96 55.88) (size 0.8) (drill 0.4) (layers "F.Cu" "B.Cu") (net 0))
 (via (at 86.36 50.8) (size 0.8) (drill 0.4) (layers "F.Cu" "B.Cu") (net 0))
 (via (at 71.12 50.8) (size 0.8) (drill 0.4) (layers "F.Cu" "B.Cu") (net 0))
 (via (at 60.96 43.18) (size 0.8) (drill 0.4) (layers "F.Cu" "B.Cu") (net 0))
 (via (at 63.5 43.18) (size 0.8) (drill 0.4) (layers "F.Cu" "B.Cu") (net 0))
 (via (at 55.88 35.56) (size 0.8) (drill 0.4) (layers "F.Cu" "B.Cu") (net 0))
 (via (at 88.9 40.64) (size 0.8) (drill 0.4) (layers "F.Cu" "B.Cu") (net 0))
 (via (at 81.28 50.8) (size 0.8) (drill 0.4) (layers "F.Cu" "B.Cu") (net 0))
 (via (at 55.88 53.34) (size 0.8) (drill 0.4) (layers "F.Cu" "B.Cu") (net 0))
 (via (at 71.12 55.88) (size 0.8) (drill 0.4) (layers "F.Cu" "B.Cu") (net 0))
 (via (at 55.88 45.72) (size 0.8) (drill 0.4) (layers "F.Cu" "B.Cu") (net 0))
 (via (at 60.96 53.34) (size 0.8) (drill 0.4) (layers "F.Cu" "B.Cu") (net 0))
 (via (at 76.2 50.8) (size 0.8) (drill 0.4) (layers "F.Cu" "B.Cu") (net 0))
 (via (at 71.12 45.72) (size 0.8) (drill 0.4) (layers "F.Cu" "B.Cu") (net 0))
 (via (at 55.88 38.1) (size 0.8) (drill 0.4) (layers "F.Cu" "B.Cu") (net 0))
 (via (at 66.04 53.34) (size 0.8) (drill 0.4) (layers "F.Cu" "B.Cu") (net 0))
 (via (at 53.34 53.34) (size 0.8) (drill 0.4) (layers "F.Cu" "B.Cu") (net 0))
 (via (at 71.12 35.56) (size 0.8) (drill 0.4) (layers "F.Cu" "B.Cu") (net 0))
 (via (at 78.74 50.8) (size 0.8) (drill 0.4) (layers "F.Cu" "B.Cu") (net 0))
 (via (at 58.42 45.72) (size 0.8) (drill 0.4) (layers "F.Cu" "B.Cu") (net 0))
 (via (at 76.2 48.26) (size 0.8) (drill 0.4) (layers "F.Cu" "B.Cu") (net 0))
 (via (at 86.36 48.26) (size 0.8) (drill 0.4) (layers "F.Cu" "B.Cu") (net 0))
 (via (at 76.2 33.02) (size 0.8) (drill 0.4) (layers "F.Cu" "B.Cu") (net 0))
 (segment (start 83.82 35.56) (end 83.82 43.18) (width 0.25) (layer "B.Cu") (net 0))
 (segment (start 68.58 35.56) (end 68.58 33.02) (width 0.25) (layer "B.Cu") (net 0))
 (segment (start 73.66 33.02) (end 71.12 33.02) (width 0.25) (layer "B.Cu") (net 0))
 (segment (start 58.42 35.56) (end 58.42 33.02) (width 0.25) (layer "B.Cu") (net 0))
 (segment (start 71.12 33.02) (end 68.58 33.02) (width 0.25) (layer "B.Cu") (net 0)))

